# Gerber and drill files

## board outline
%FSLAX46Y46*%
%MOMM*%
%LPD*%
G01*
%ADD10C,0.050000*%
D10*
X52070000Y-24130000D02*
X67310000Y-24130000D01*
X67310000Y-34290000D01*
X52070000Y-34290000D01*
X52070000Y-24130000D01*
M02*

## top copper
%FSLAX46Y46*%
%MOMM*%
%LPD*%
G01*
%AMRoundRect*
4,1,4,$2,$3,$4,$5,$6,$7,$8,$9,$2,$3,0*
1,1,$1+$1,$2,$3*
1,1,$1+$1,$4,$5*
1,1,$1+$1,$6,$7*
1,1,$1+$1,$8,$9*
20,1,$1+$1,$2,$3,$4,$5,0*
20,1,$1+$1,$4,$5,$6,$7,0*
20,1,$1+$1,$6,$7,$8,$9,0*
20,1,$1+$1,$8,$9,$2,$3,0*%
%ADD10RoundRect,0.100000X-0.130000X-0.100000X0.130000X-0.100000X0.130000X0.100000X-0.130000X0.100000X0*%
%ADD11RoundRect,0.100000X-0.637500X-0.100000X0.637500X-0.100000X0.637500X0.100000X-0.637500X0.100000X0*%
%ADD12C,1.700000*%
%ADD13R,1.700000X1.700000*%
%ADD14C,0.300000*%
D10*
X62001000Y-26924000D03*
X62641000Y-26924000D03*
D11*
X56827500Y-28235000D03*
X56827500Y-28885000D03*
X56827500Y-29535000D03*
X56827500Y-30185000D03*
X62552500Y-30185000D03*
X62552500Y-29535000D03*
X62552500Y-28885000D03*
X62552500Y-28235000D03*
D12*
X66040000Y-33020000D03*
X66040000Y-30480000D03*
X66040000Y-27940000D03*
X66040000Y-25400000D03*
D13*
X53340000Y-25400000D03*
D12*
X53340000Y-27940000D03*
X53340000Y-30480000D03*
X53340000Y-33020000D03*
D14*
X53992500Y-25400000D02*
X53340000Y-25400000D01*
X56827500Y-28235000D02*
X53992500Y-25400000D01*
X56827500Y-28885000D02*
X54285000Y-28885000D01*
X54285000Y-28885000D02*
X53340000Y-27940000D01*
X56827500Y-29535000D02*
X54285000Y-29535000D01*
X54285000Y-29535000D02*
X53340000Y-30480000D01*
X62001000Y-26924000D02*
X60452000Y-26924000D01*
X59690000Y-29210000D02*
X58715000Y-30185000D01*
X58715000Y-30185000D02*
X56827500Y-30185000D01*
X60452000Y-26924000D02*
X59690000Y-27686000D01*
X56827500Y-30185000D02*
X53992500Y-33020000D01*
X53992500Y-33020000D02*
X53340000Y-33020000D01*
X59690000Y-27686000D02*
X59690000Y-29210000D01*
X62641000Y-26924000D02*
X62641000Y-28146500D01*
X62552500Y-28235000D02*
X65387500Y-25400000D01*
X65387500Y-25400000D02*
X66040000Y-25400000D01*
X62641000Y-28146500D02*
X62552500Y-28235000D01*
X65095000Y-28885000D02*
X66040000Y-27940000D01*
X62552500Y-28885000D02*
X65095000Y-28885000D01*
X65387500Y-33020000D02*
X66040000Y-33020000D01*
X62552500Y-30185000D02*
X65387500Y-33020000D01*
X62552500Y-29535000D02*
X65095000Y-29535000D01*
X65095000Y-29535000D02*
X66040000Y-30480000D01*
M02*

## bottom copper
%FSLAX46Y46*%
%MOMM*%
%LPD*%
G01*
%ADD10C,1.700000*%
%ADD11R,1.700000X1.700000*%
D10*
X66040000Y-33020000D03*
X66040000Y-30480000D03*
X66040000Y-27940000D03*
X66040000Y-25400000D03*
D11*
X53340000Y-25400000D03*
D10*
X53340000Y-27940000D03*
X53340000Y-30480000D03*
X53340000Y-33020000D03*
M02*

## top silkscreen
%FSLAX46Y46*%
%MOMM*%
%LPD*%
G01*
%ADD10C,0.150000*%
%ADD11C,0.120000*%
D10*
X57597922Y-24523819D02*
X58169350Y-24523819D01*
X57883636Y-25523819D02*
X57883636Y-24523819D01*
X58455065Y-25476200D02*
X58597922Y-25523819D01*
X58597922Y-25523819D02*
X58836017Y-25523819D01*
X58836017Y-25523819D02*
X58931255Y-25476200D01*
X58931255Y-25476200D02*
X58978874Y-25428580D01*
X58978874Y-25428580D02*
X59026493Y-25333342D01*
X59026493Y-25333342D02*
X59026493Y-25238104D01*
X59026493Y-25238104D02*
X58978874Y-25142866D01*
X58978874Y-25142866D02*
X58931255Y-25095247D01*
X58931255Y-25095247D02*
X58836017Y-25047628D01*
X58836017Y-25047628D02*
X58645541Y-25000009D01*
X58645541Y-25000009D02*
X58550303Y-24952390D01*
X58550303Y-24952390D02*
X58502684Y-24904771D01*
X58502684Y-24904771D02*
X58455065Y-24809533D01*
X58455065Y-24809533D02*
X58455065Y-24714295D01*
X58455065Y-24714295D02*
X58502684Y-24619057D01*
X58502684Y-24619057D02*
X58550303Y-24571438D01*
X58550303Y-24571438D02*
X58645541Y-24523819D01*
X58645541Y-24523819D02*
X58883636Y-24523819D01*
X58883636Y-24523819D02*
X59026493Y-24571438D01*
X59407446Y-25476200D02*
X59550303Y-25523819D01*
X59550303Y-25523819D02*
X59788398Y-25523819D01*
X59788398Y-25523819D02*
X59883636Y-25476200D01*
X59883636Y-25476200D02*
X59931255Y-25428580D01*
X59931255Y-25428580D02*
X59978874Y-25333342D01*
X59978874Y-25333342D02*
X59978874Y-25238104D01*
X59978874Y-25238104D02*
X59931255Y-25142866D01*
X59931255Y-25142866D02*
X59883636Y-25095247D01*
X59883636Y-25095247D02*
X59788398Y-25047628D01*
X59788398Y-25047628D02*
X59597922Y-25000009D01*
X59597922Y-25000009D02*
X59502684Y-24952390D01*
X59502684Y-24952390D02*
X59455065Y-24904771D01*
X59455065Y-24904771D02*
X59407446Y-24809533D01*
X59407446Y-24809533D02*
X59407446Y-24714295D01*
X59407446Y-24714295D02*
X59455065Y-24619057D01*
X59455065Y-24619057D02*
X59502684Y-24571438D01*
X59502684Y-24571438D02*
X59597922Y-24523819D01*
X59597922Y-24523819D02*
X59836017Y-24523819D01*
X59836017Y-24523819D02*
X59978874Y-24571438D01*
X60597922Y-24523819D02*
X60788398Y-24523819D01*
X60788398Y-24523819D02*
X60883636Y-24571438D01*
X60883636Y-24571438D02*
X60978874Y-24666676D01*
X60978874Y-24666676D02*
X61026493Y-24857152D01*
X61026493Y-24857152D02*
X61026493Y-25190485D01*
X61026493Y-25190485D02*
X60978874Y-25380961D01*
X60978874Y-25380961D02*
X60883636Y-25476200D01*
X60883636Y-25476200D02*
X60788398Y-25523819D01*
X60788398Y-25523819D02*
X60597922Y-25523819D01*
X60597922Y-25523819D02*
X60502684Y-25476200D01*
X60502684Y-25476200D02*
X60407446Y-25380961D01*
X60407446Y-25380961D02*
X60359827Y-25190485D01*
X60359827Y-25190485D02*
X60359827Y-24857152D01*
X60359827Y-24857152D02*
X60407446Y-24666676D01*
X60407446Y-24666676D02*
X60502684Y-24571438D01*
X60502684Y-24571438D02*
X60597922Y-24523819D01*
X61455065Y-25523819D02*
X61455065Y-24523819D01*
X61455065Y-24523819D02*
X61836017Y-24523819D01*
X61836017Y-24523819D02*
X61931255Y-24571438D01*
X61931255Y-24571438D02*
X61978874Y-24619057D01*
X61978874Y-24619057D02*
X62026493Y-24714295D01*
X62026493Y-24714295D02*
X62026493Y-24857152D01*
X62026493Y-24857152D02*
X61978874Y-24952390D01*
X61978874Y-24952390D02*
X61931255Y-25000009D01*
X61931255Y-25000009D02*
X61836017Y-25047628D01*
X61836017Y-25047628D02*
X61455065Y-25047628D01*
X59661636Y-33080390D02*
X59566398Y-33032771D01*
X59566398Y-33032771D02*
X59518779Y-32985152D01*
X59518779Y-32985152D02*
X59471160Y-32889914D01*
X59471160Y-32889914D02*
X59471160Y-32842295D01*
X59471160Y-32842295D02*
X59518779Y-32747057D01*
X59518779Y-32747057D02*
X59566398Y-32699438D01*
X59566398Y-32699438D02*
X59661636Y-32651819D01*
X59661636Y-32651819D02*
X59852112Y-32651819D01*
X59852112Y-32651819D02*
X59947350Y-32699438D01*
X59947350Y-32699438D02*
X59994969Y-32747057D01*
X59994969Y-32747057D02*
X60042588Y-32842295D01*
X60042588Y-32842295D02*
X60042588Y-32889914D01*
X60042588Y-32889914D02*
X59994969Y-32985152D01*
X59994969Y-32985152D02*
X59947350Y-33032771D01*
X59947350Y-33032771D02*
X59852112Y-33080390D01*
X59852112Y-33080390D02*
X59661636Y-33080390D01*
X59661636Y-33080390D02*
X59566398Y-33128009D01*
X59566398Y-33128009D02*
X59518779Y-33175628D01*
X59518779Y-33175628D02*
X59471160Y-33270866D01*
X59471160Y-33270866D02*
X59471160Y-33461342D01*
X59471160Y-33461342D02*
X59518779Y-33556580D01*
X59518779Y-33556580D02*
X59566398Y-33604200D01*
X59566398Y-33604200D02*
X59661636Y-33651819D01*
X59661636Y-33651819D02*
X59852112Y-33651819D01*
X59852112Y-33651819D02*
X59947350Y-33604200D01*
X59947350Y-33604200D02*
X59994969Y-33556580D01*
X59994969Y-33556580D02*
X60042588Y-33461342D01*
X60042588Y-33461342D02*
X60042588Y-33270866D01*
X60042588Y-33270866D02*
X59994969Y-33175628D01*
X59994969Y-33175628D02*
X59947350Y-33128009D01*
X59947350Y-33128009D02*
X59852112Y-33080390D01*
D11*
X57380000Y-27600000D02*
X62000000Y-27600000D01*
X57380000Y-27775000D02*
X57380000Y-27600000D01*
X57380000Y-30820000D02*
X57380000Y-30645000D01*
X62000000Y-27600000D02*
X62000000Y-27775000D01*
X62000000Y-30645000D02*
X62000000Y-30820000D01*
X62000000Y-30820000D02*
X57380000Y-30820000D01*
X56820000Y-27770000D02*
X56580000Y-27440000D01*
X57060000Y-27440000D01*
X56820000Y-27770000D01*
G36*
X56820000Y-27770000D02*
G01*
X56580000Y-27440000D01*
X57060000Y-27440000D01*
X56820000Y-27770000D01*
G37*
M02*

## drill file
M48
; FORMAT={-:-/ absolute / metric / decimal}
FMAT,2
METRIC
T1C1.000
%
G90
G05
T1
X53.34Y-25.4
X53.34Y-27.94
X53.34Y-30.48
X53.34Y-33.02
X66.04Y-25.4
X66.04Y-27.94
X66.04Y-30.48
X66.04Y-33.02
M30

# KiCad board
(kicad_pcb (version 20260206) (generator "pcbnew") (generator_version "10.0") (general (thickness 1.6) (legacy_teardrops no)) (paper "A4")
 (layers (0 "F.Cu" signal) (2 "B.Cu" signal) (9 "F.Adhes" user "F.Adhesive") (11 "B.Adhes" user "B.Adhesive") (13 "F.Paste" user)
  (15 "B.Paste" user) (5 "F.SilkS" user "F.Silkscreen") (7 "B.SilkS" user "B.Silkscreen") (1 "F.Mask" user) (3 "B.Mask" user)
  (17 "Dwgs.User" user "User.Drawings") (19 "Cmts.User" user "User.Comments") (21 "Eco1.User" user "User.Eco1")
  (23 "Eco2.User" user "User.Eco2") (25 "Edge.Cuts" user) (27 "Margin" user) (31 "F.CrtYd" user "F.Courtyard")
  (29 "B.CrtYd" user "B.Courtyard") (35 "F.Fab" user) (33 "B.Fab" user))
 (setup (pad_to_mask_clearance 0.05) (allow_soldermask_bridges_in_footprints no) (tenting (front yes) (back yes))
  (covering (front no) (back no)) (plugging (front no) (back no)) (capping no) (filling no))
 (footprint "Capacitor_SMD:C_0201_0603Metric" (layer "F.Cu") (at 62.321 26.924)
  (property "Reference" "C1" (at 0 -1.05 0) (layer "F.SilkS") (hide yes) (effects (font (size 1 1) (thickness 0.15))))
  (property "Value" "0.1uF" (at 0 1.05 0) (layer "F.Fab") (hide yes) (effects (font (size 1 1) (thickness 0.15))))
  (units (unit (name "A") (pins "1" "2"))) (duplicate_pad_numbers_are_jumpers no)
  (pad "" smd roundrect (at -0.345 0) (size 0.318 0.36) (layers "F.Paste") (roundrect_rratio 0.25))
  (pad "" smd roundrect (at 0.345 0) (size 0.318 0.36) (layers "F.Paste") (roundrect_rratio 0.25))
  (pad "1" smd roundrect (at -0.32 0) (size 0.46 0.4) (layers "F.Cu" "F.Mask") (roundrect_rratio 0.25) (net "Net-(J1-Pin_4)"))
  (pad "2" smd roundrect (at 0.32 0) (size 0.46 0.4) (layers "F.Cu" "F.Mask") (roundrect_rratio 0.25) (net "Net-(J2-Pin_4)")))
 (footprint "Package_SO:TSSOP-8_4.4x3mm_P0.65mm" (layer "F.Cu") (at 59.69 29.21)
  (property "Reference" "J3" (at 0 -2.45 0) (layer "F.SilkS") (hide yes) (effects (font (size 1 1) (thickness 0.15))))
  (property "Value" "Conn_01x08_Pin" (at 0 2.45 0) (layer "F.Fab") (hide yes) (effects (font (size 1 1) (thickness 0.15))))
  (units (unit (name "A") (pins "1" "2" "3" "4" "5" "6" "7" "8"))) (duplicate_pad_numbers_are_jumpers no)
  (fp_line (start -2.31 -1.61) (end 2.31 -1.61) (stroke (width 0.12) (type solid)) (layer "F.SilkS"))
  (fp_line (start -2.31 -1.435) (end -2.31 -1.61) (stroke (width 0.12) (type solid)) (layer "F.SilkS"))
  (fp_line (start -2.31 1.61) (end -2.31 1.435) (stroke (width 0.12) (type solid)) (layer "F.SilkS"))
  (fp_line (start 2.31 -1.61) (end 2.31 -1.435) (stroke (width 0.12) (type solid)) (layer "F.SilkS"))
  (fp_line (start 2.31 1.435) (end 2.31 1.61) (stroke (width 0.12) (type solid)) (layer "F.SilkS"))
  (fp_line (start 2.31 1.61) (end -2.31 1.61) (stroke (width 0.12) (type solid)) (layer "F.SilkS"))
  (fp_poly (pts (xy -2.87 -1.44) (xy -3.11 -1.77) (xy -2.63 -1.77)) (stroke (width 0.12) (type solid)) (fill yes) (layer "F.SilkS"))
  (pad "1" smd roundrect (at -2.8625 -0.975) (size 1.475 0.4) (layers "F.Cu" "F.Mask" "F.Paste") (roundrect_rratio 0.25)
   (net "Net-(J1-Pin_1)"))
  (pad "2" smd roundrect (at -2.8625 -0.325) (size 1.475 0.4) (layers "F.Cu" "F.Mask" "F.Paste") (roundrect_rratio 0.25)
   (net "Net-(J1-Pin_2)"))
  (pad "3" smd roundrect (at -2.8625 0.325) (size 1.475 0.4) (layers "F.Cu" "F.Mask" "F.Paste") (roundrect_rratio 0.25)
   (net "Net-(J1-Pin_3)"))
  (pad "4" smd roundrect (at -2.8625 0.975) (size 1.475 0.4) (layers "F.Cu" "F.Mask" "F.Paste") (roundrect_rratio 0.25)
   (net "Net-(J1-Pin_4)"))
  (pad "5" smd roundrect (at 2.8625 0.975) (size 1.475 0.4) (layers "F.Cu" "F.Mask" "F.Paste") (roundrect_rratio 0.25)
   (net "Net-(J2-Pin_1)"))
  (pad "6" smd roundrect (at 2.8625 0.325) (size 1.475 0.4) (layers "F.Cu" "F.Mask" "F.Paste") (roundrect_rratio 0.25)
   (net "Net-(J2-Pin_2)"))
  (pad "7" smd roundrect (at 2.8625 -0.325) (size 1.475 0.4) (layers "F.Cu" "F.Mask" "F.Paste") (roundrect_rratio 0.25)
   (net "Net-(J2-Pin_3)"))
  (pad "8" smd roundrect (at 2.8625 -0.975) (size 1.475 0.4) (layers "F.Cu" "F.Mask" "F.Paste") (roundrect_rratio 0.25)
   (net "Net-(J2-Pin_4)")))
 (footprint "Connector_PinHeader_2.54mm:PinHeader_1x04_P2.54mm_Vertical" (layer "B.Cu") (at 66.04 33.02)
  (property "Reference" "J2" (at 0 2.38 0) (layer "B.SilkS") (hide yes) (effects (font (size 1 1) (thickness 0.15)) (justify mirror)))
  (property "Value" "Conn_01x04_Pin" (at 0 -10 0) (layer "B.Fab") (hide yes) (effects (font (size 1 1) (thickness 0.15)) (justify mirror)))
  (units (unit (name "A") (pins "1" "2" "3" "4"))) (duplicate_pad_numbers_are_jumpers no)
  (pad "1" thru_hole circle (at 0 0) (size 1.7 1.7) (drill 1) (layers "*.Cu" "*.Mask") (remove_unused_layers no) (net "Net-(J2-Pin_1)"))
  (pad "2" thru_hole circle (at 0 -2.54) (size 1.7 1.7) (drill 1) (layers "*.Cu" "*.Mask") (remove_unused_layers no) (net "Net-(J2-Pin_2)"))
  (pad "3" thru_hole circle (at 0 -5.08) (size 1.7 1.7) (drill 1) (layers "*.Cu" "*.Mask") (remove_unused_layers no) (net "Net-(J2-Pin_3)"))
  (pad "4" thru_hole circle (at 0 -7.62) (size 1.7 1.7) (drill 1) (layers "*.Cu" "*.Mask") (remove_unused_layers no) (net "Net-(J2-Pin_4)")))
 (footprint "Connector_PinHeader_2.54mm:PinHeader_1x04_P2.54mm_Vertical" (layer "B.Cu") (at 53.34 25.4 180)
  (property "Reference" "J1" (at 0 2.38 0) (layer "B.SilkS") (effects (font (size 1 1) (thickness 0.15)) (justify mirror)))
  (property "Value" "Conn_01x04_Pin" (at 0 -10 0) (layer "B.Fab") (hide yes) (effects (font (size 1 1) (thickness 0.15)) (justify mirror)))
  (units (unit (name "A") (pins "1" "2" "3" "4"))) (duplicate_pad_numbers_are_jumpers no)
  (pad "1" thru_hole rect (at 0 0 180) (size 1.7 1.7) (drill 1) (layers "*.Cu" "*.Mask") (remove_unused_layers no) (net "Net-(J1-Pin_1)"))
  (pad "2" thru_hole circle (at 0 -2.54 180) (size 1.7 1.7) (drill 1) (layers "*.Cu" "*.Mask") (remove_unused_layers no)
   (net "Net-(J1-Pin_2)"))
  (pad "3" thru_hole circle (at 0 -5.08 180) (size 1.7 1.7) (drill 1) (layers "*.Cu" "*.Mask") (remove_unused_layers no)
   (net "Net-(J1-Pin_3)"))
  (pad "4" thru_hole circle (at 0 -7.62 180) (size 1.7 1.7) (drill 1) (layers "*.Cu" "*.Mask") (remove_unused_layers no)
   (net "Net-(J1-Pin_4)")))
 (gr_rect (start 52.07 24.13) (end 67.31 34.29) (stroke (width 0.05) (type default)) (fill no) (layer "Edge.Cuts"))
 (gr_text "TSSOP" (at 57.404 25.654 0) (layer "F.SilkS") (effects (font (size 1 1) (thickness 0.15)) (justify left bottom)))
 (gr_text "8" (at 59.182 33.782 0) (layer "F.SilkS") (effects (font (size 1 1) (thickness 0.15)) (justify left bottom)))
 (segment (start 53.9925 25.4) (end 53.34 25.4) (width 0.3) (layer "F.Cu") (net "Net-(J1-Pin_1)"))
 (segment (start 56.8275 28.235) (end 53.9925 25.4) (width 0.3) (layer "F.Cu") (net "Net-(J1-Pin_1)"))
 (segment (start 56.8275 28.885) (end 54.285 28.885) (width 0.3) (layer "F.Cu") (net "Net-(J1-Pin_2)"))
 (segment (start 54.285 28.885) (end 53.34 27.94) (width 0.3) (layer "F.Cu") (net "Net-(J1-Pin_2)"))
 (segment (start 56.8275 29.535) (end 54.285 29.535) (width 0.3) (layer "F.Cu") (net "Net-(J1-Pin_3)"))
 (segment (start 54.285 29.535) (end 53.34 30.48) (width 0.3) (layer "F.Cu") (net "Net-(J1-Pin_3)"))
 (segment (start 62.001 26.924) (end 60.452 26.924) (width 0.3) (layer "F.Cu") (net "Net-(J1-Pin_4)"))
 (segment (start 59.69 29.21) (end 58.715 30.185) (width 0.3) (layer "F.Cu") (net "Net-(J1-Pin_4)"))
 (segment (start 58.715 30.185) (end 56.8275 30.185) (width 0.3) (layer "F.Cu") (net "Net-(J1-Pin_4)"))
 (segment (start 60.452 26.924) (end 59.69 27.686) (width 0.3) (layer "F.Cu") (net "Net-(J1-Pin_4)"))
 (segment (start 56.8275 30.185) (end 53.9925 33.02) (width 0.3) (layer "F.Cu") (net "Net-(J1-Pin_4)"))
 (segment (start 53.9925 33.02) (end 53.34 33.02) (width 0.3) (layer "F.Cu") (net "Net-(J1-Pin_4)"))
 (segment (start 59.69 27.686) (end 59.69 29.21) (width 0.3) (layer "F.Cu") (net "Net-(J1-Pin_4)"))
 (segment (start 62.641 26.924) (end 62.641 28.1465) (width 0.3) (layer "F.Cu") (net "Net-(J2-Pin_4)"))
 (segment (start 62.5525 28.235) (end 65.3875 25.4) (width 0.3) (layer "F.Cu") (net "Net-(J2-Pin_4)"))
 (segment (start 65.3875 25.4) (end 66.04 25.4) (width 0.3) (layer "F.Cu") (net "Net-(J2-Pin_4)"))
 (segment (start 62.641 28.1465) (end 62.5525 28.235) (width 0.3) (layer "F.Cu") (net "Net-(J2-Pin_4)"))
 (segment (start 65.095 28.885) (end 66.04 27.94) (width 0.3) (layer "F.Cu") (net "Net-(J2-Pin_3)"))
 (segment (start 62.5525 28.885) (end 65.095 28.885) (width 0.3) (layer "F.Cu") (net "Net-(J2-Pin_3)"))
 (segment (start 65.3875 33.02) (end 66.04 33.02) (width 0.3) (layer "F.Cu") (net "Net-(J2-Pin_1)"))
 (segment (start 62.5525 30.185) (end 65.3875 33.02) (width 0.3) (layer "F.Cu") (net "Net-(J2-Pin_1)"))
 (segment (start 62.5525 29.535) (end 65.095 29.535) (width 0.3) (layer "F.Cu") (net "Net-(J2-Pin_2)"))
 (segment (start 65.095 29.535) (end 66.04 30.48) (width 0.3) (layer "F.Cu") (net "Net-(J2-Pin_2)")))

